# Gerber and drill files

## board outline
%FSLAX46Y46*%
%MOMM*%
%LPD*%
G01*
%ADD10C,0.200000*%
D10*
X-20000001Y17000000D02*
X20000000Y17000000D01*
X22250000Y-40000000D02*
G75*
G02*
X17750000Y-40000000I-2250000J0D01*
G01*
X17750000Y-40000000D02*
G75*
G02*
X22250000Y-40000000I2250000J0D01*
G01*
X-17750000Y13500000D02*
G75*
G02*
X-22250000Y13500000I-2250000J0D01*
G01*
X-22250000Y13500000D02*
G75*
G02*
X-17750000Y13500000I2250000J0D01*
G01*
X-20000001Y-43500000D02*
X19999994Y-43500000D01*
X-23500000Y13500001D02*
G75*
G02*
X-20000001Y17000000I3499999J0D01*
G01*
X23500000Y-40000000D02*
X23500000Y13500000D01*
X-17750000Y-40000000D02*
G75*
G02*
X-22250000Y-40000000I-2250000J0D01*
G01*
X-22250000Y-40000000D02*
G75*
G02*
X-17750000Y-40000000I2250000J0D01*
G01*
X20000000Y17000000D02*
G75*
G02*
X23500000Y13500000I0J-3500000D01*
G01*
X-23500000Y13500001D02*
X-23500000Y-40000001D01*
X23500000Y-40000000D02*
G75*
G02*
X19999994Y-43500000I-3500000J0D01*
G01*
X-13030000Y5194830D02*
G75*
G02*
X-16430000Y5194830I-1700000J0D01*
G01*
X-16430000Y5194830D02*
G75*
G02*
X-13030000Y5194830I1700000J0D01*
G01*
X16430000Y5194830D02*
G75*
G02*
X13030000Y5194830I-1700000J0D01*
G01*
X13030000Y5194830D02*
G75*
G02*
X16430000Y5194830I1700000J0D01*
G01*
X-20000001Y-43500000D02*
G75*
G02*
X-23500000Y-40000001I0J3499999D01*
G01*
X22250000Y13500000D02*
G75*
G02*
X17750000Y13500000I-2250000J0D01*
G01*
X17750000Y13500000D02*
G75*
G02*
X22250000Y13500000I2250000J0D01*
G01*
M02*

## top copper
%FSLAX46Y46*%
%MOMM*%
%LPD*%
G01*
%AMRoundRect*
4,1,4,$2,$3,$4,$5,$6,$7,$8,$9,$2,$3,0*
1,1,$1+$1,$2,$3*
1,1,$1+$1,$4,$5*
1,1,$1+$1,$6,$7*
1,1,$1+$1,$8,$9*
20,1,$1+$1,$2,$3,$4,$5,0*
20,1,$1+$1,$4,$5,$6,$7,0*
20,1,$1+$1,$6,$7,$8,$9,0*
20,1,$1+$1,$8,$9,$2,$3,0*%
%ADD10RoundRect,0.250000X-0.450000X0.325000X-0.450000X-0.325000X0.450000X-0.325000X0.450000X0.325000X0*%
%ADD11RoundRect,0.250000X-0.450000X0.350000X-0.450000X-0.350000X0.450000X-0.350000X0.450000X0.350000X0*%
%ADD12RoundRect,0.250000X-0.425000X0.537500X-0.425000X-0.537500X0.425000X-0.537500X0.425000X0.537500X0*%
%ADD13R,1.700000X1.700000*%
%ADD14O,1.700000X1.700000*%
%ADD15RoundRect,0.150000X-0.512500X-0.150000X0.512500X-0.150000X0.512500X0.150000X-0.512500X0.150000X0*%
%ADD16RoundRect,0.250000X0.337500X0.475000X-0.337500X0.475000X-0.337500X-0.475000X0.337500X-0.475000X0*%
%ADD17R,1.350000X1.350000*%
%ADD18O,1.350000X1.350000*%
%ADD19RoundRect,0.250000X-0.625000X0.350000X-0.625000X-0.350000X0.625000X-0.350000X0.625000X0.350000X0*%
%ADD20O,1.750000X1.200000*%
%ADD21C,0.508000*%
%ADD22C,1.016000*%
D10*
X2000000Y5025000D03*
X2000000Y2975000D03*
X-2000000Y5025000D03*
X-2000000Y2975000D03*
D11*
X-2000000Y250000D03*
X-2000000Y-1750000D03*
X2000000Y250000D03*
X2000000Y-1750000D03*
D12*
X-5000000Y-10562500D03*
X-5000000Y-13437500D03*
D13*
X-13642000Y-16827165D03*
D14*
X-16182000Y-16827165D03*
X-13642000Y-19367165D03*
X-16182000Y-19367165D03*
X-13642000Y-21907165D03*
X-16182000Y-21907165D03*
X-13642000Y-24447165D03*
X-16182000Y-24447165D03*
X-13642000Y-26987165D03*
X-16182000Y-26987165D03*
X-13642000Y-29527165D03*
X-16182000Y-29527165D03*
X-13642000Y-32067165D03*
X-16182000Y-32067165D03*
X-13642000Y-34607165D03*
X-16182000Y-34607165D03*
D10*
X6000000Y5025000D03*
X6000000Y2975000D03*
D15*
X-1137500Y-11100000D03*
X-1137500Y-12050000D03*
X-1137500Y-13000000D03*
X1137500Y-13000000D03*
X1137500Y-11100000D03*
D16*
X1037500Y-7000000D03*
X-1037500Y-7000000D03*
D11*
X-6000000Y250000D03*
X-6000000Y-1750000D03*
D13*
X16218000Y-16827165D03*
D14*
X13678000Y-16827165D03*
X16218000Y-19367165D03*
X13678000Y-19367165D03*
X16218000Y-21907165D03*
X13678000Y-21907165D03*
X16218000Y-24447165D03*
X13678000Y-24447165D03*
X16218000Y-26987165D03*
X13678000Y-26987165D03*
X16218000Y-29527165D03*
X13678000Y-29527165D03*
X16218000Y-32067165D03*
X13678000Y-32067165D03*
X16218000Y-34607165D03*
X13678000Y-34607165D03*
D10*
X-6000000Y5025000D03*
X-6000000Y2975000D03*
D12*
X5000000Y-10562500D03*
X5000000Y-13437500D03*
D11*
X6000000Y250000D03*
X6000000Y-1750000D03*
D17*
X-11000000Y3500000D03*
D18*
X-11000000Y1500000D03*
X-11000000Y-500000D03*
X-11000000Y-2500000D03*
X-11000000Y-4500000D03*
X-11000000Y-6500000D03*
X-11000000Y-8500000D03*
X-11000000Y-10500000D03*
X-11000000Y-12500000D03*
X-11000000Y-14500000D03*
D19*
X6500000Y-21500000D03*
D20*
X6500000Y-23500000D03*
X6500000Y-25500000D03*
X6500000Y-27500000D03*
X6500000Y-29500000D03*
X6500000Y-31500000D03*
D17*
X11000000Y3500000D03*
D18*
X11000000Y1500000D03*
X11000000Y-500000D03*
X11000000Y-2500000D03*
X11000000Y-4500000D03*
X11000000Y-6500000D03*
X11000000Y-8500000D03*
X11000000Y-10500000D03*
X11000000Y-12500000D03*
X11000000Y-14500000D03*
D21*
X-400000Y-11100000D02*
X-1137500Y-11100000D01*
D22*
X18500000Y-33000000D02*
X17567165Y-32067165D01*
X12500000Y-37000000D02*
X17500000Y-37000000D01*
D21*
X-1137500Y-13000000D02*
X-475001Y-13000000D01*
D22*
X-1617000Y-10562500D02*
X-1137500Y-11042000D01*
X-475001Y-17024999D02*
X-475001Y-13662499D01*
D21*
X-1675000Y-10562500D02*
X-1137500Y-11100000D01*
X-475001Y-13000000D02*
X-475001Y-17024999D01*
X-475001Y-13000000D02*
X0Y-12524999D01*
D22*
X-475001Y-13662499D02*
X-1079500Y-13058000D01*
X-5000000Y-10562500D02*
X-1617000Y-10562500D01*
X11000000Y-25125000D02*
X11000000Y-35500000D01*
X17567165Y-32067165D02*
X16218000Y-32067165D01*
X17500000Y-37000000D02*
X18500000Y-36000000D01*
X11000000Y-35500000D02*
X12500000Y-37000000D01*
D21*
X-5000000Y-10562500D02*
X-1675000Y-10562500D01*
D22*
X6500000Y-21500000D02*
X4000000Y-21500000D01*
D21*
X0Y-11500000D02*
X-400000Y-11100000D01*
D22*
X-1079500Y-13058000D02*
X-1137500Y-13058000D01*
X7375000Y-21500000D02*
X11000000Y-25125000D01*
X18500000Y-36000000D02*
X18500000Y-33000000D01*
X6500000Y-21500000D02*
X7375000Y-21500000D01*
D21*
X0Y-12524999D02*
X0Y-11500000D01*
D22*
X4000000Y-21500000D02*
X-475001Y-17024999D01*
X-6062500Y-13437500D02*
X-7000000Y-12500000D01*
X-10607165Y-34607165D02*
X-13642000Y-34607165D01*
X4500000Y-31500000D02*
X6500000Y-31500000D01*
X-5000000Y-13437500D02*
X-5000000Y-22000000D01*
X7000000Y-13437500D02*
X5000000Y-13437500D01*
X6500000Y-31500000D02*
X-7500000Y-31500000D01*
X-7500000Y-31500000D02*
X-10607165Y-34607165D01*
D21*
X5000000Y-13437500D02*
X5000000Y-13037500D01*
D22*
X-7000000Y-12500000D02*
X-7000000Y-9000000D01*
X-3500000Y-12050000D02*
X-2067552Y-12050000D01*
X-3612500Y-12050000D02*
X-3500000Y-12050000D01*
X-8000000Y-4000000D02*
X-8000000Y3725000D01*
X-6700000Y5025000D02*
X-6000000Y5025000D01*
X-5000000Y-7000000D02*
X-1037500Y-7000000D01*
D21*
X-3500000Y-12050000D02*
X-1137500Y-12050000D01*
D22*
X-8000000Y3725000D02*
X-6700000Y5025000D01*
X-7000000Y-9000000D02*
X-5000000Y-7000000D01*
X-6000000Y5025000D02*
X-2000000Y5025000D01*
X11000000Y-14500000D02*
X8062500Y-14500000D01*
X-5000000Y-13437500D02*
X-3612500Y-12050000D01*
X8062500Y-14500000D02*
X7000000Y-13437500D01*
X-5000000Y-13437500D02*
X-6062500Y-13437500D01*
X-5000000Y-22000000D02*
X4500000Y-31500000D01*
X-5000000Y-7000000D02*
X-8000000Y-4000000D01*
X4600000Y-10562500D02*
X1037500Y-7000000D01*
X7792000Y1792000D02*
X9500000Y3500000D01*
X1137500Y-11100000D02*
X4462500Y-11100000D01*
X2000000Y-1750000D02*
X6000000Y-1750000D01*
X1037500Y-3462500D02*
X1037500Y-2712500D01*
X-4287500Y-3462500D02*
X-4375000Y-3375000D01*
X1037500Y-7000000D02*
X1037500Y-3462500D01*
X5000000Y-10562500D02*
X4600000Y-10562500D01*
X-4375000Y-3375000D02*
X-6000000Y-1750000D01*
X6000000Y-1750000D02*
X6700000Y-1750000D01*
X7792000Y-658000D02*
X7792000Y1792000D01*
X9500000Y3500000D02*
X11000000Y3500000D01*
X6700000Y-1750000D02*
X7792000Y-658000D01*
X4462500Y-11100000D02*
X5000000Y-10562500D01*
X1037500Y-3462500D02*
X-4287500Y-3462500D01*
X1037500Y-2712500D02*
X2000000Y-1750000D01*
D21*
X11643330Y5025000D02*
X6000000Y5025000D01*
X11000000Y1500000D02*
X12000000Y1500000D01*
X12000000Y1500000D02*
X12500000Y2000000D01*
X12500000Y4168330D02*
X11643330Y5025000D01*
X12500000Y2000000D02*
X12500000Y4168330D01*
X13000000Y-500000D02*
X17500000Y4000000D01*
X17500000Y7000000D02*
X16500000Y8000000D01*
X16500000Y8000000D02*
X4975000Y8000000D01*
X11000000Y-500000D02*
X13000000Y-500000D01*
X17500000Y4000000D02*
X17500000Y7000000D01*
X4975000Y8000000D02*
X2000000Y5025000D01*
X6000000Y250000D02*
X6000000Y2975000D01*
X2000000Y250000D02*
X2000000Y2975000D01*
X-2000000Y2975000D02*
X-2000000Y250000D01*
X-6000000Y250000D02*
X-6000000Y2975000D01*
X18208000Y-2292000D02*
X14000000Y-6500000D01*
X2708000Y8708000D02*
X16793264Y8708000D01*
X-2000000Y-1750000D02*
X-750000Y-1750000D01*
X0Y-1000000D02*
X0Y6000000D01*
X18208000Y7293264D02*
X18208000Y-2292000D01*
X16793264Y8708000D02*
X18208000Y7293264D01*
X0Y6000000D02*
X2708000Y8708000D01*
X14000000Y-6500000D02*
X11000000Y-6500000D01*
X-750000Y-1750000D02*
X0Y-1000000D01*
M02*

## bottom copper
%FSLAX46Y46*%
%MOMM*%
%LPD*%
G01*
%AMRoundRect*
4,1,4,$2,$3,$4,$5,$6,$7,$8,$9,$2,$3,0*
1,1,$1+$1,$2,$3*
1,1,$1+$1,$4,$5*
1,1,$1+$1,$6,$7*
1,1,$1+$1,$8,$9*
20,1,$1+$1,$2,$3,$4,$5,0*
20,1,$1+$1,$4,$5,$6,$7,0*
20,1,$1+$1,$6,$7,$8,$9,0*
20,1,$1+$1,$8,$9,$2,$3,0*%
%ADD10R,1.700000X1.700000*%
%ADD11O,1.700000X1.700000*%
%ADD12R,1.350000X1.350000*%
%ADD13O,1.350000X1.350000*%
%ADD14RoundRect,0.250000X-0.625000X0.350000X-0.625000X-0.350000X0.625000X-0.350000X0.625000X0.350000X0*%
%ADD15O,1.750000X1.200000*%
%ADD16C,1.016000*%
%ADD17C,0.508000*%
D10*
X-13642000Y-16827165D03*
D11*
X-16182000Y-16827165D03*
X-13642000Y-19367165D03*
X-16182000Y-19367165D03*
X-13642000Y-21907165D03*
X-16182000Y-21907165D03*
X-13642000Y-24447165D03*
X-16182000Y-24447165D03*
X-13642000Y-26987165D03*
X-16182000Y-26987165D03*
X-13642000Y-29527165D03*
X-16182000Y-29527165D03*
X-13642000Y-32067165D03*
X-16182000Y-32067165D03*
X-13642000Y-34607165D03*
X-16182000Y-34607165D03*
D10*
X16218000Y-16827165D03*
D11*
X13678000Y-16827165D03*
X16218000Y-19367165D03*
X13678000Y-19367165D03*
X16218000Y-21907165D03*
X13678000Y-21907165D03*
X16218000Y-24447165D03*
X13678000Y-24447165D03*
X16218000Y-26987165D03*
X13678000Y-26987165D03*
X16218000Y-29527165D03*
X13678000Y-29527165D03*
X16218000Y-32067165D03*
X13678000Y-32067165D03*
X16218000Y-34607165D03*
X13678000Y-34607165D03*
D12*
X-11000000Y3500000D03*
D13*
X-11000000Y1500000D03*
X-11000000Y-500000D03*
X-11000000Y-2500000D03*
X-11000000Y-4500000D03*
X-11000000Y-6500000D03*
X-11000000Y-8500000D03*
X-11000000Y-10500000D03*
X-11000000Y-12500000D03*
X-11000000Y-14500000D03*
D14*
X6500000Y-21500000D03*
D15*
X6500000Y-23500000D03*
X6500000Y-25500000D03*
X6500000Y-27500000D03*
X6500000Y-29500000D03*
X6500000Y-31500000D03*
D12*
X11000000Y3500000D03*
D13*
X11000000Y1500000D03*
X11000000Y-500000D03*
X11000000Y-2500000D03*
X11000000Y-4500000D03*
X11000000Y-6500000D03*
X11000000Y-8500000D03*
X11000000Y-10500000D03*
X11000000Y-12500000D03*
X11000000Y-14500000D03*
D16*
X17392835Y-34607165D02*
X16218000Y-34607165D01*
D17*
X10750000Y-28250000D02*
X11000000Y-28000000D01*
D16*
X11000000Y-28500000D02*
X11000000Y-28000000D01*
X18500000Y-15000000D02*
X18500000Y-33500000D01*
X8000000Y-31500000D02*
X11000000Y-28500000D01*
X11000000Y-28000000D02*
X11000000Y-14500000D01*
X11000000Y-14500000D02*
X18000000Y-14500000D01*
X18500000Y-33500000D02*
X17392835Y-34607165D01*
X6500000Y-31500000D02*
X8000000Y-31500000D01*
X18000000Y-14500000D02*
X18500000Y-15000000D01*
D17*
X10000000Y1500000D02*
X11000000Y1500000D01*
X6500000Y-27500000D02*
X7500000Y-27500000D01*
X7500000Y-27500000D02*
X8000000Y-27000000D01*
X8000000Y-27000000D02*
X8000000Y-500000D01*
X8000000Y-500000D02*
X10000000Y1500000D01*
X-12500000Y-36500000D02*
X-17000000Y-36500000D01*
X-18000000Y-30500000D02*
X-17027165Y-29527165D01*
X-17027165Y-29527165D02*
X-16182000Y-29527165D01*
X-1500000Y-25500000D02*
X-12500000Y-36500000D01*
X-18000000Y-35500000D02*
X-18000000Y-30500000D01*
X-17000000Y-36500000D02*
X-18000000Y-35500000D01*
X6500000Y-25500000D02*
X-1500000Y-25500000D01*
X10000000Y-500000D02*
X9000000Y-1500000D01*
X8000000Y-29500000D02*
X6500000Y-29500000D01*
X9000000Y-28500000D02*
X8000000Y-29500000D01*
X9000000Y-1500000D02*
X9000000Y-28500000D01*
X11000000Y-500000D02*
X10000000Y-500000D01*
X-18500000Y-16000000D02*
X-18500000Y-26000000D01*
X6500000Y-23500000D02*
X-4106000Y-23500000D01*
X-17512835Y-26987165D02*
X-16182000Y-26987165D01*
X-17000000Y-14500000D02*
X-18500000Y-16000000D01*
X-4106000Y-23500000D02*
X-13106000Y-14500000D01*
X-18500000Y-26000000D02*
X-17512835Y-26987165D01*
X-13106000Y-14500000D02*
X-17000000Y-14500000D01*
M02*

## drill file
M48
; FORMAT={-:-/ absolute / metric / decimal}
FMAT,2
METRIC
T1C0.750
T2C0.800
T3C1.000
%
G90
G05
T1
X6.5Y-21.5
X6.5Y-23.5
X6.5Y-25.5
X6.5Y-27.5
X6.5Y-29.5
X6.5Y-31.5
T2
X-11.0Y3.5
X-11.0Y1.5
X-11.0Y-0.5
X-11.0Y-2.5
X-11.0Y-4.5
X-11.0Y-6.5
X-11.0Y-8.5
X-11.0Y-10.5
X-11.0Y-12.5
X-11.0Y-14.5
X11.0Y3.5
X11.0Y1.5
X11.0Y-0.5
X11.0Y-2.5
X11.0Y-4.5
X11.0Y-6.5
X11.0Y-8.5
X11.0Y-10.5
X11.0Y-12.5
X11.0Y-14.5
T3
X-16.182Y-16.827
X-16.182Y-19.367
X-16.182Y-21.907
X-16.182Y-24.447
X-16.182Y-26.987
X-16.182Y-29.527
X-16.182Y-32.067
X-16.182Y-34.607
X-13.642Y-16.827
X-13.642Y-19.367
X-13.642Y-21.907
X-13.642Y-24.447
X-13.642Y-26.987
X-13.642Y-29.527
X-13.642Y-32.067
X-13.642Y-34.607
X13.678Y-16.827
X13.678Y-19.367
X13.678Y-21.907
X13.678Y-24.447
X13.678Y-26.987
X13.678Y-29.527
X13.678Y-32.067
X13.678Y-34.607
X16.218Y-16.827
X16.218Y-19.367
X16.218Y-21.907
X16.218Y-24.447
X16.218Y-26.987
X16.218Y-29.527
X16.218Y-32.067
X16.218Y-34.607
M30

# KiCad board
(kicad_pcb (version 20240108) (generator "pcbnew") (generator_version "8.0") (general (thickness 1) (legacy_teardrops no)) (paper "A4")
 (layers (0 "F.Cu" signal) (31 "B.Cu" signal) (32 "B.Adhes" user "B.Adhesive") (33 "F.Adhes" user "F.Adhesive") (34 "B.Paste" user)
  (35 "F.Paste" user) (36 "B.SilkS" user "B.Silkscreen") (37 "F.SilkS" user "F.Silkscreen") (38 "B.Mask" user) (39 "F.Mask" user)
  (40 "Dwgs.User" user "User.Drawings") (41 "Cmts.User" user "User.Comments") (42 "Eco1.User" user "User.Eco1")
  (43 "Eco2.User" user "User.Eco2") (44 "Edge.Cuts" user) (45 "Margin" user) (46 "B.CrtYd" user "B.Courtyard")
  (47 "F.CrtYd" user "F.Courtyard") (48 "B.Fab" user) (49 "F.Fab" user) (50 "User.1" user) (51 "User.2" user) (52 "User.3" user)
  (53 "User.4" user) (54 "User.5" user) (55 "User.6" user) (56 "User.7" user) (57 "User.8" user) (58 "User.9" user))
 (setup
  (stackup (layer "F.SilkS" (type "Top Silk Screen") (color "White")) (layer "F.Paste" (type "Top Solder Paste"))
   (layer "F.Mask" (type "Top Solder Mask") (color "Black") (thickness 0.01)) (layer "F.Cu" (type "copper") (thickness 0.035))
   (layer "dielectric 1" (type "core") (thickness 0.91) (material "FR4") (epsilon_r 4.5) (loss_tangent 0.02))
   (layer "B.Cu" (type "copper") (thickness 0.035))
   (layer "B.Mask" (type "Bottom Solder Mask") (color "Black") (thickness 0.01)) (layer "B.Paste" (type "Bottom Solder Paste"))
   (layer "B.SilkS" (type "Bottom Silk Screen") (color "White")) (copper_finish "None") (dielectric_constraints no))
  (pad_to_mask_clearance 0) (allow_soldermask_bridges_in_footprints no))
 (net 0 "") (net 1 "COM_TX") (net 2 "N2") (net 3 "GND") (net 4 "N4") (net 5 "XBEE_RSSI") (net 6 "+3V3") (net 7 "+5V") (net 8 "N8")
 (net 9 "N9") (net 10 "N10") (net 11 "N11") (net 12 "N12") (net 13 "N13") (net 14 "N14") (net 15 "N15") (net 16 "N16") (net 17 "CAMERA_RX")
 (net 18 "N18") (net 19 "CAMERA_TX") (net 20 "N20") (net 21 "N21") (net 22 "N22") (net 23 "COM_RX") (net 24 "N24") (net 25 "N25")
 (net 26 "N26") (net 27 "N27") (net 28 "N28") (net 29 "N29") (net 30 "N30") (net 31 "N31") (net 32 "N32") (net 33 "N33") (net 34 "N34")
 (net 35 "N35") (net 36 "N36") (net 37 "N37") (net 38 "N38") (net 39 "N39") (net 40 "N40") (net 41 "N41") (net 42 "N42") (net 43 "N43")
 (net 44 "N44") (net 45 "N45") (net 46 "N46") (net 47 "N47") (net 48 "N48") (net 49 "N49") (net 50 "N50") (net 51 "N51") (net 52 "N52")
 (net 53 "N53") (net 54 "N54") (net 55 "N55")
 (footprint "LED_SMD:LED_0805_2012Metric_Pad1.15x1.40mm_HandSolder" (layer "F.Cu") (at 2 -4 -90)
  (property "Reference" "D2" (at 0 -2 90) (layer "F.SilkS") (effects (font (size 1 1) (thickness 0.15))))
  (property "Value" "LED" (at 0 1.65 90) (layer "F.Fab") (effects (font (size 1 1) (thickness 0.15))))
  (pad "1" smd roundrect (at -1.025 0 270) (size 1.15 1.4) (layers "F.Cu" "F.Paste" "F.Mask") (roundrect_rratio 0.217391) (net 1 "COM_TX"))
  (pad "2" smd roundrect (at 1.025 0 270) (size 1.15 1.4) (layers "F.Cu" "F.Paste" "F.Mask") (roundrect_rratio 0.217391) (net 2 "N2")))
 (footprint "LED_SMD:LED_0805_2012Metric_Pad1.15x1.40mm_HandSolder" (layer "F.Cu") (at -2 -4 -90)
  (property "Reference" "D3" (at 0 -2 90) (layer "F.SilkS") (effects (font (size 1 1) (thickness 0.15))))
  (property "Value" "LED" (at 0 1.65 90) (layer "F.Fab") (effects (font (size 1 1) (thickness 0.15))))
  (pad "1" smd roundrect (at -1.025 0 270) (size 1.15 1.4) (layers "F.Cu" "F.Paste" "F.Mask") (roundrect_rratio 0.217391) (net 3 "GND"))
  (pad "2" smd roundrect (at 1.025 0 270) (size 1.15 1.4) (layers "F.Cu" "F.Paste" "F.Mask") (roundrect_rratio 0.217391) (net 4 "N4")))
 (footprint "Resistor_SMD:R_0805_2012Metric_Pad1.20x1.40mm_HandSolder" (layer "F.Cu") (at -2 0.75 -90)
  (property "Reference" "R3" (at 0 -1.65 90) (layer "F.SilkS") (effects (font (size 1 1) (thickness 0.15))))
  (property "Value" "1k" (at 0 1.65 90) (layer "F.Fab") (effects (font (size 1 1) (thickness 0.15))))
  (pad "1" smd roundrect (at -1 0 270) (size 1.2 1.4) (layers "F.Cu" "F.Paste" "F.Mask") (roundrect_rratio 0.208333) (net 4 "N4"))
  (pad "2" smd roundrect (at 1 0 270) (size 1.2 1.4) (layers "F.Cu" "F.Paste" "F.Mask") (roundrect_rratio 0.208333) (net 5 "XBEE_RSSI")))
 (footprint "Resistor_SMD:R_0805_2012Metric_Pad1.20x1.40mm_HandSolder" (layer "F.Cu") (at 2 0.75 -90)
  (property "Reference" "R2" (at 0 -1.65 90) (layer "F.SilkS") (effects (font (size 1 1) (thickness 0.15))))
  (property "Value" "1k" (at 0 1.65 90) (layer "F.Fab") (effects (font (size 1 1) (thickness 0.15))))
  (pad "1" smd roundrect (at -1 0 270) (size 1.2 1.4) (layers "F.Cu" "F.Paste" "F.Mask") (roundrect_rratio 0.208333) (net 2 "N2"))
  (pad "2" smd roundrect (at 1 0 270) (size 1.2 1.4) (layers "F.Cu" "F.Paste" "F.Mask") (roundrect_rratio 0.208333) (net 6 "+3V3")))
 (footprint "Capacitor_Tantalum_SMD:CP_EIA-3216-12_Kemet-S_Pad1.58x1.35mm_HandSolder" (layer "F.Cu") (at -5 12 -90)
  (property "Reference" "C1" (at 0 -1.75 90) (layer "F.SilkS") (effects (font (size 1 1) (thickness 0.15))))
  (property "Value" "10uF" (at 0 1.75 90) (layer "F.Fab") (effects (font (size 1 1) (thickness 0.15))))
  (pad "1" smd roundrect (at -1.4375 0 270) (size 1.575 1.35) (layers "F.Cu" "F.Paste" "F.Mask") (roundrect_rratio 0.185185) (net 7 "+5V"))
  (pad "2" smd roundrect (at 1.4375 0 270) (size 1.575 1.35) (layers "F.Cu" "F.Paste" "F.Mask") (roundrect_rratio 0.185185) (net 3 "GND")))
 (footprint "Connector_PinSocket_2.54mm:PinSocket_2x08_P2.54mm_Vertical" (layer "F.Cu") (at -13.642 16.827165)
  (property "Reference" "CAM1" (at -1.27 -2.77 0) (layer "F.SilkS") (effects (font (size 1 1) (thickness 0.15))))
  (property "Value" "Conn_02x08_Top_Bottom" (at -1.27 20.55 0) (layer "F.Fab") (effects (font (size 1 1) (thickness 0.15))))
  (pad "1" thru_hole rect (at 0 0) (size 1.7 1.7) (drill 1) (layers "*.Cu" "*.Mask") (remove_unused_layers no) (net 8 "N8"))
  (pad "2" thru_hole oval (at -2.54 0) (size 1.7 1.7) (drill 1) (layers "*.Cu" "*.Mask") (remove_unused_layers no) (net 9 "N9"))
  (pad "3" thru_hole oval (at 0 2.54) (size 1.7 1.7) (drill 1) (layers "*.Cu" "*.Mask") (remove_unused_layers no) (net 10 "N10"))
  (pad "4" thru_hole oval (at -2.54 2.54) (size 1.7 1.7) (drill 1) (layers "*.Cu" "*.Mask") (remove_unused_layers no) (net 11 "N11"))
  (pad "5" thru_hole oval (at 0 5.08) (size 1.7 1.7) (drill 1) (layers "*.Cu" "*.Mask") (remove_unused_layers no) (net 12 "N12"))
  (pad "6" thru_hole oval (at -2.54 5.08) (size 1.7 1.7) (drill 1) (layers "*.Cu" "*.Mask") (remove_unused_layers no) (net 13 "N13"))
  (pad "7" thru_hole oval (at 0 7.62) (size 1.7 1.7) (drill 1) (layers "*.Cu" "*.Mask") (remove_unused_layers no) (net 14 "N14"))
  (pad "8" thru_hole oval (at -2.54 7.62) (size 1.7 1.7) (drill 1) (layers "*.Cu" "*.Mask") (remove_unused_layers no) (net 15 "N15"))
  (pad "9" thru_hole oval (at 0 10.16) (size 1.7 1.7) (drill 1) (layers "*.Cu" "*.Mask") (remove_unused_layers no) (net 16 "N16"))
  (pad "10" thru_hole oval (at -2.54 10.16) (size 1.7 1.7) (drill 1) (layers "*.Cu" "*.Mask") (remove_unused_layers no) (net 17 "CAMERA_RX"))
  (pad "11" thru_hole oval (at 0 12.7) (size 1.7 1.7) (drill 1) (layers "*.Cu" "*.Mask") (remove_unused_layers no) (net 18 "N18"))
  (pad "12" thru_hole oval (at -2.54 12.7) (size 1.7 1.7) (drill 1) (layers "*.Cu" "*.Mask") (remove_unused_layers no) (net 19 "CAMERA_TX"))
  (pad "13" thru_hole oval (at 0 15.24) (size 1.7 1.7) (drill 1) (layers "*.Cu" "*.Mask") (remove_unused_layers no) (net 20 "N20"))
  (pad "14" thru_hole oval (at -2.54 15.24) (size 1.7 1.7) (drill 1) (layers "*.Cu" "*.Mask") (remove_unused_layers no) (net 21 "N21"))
  (pad "15" thru_hole oval (at 0 17.78) (size 1.7 1.7) (drill 1) (layers "*.Cu" "*.Mask") (remove_unused_layers no) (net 3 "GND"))
  (pad "16" thru_hole oval (at -2.54 17.78) (size 1.7 1.7) (drill 1) (layers "*.Cu" "*.Mask") (remove_unused_layers no) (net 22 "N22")))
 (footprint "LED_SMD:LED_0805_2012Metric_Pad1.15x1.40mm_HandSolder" (layer "F.Cu") (at 6 -4 -90)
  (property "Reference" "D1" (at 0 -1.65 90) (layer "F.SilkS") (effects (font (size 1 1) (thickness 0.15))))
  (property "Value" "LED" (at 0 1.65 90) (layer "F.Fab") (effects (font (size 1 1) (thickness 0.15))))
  (pad "1" smd roundrect (at -1.025 0 270) (size 1.15 1.4) (layers "F.Cu" "F.Paste" "F.Mask") (roundrect_rratio 0.217391) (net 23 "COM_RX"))
  (pad "2" smd roundrect (at 1.025 0 270) (size 1.15 1.4) (layers "F.Cu" "F.Paste" "F.Mask") (roundrect_rratio 0.217391) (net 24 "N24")))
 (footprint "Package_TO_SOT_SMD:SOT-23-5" (layer "F.Cu") (at 0 12.05)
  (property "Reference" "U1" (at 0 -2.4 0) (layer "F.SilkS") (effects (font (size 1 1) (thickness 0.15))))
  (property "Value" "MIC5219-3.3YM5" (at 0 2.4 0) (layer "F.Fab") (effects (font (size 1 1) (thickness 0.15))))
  (pad "1" smd roundrect (at -1.1375 -0.95) (size 1.325 0.6) (layers "F.Cu" "F.Paste" "F.Mask") (roundrect_rratio 0.25) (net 7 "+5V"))
  (pad "2" smd roundrect (at -1.1375 0) (size 1.325 0.6) (layers "F.Cu" "F.Paste" "F.Mask") (roundrect_rratio 0.25) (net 3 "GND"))
  (pad "3" smd roundrect (at -1.1375 0.95) (size 1.325 0.6) (layers "F.Cu" "F.Paste" "F.Mask") (roundrect_rratio 0.25) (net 7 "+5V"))
  (pad "4" smd roundrect (at 1.1375 0.95) (size 1.325 0.6) (layers "F.Cu" "F.Paste" "F.Mask") (roundrect_rratio 0.25) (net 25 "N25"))
  (pad "5" smd roundrect (at 1.1375 -0.95) (size 1.325 0.6) (layers "F.Cu" "F.Paste" "F.Mask") (roundrect_rratio 0.25) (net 6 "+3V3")))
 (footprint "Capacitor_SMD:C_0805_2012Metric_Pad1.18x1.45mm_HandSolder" (layer "F.Cu") (at 0 7 180)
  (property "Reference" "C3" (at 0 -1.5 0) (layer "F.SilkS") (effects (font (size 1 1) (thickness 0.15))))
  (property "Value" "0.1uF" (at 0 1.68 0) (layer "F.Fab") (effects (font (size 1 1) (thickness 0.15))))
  (pad "1" smd roundrect (at -1.0375 0 180) (size 1.175 1.45) (layers "F.Cu" "F.Paste" "F.Mask") (roundrect_rratio 0.212766) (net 6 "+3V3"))
  (pad "2" smd roundrect (at 1.0375 0 180) (size 1.175 1.45) (layers "F.Cu" "F.Paste" "F.Mask") (roundrect_rratio 0.212766) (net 3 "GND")))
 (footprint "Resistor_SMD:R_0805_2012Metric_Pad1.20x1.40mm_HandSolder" (layer "F.Cu") (at -6 0.75 -90)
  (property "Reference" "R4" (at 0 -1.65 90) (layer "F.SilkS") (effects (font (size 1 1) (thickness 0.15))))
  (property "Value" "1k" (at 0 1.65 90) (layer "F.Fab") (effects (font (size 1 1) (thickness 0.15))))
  (pad "1" smd roundrect (at -1 0 270) (size 1.2 1.4) (layers "F.Cu" "F.Paste" "F.Mask") (roundrect_rratio 0.208333) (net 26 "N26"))
  (pad "2" smd roundrect (at 1 0 270) (size 1.2 1.4) (layers "F.Cu" "F.Paste" "F.Mask") (roundrect_rratio 0.208333) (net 6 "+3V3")))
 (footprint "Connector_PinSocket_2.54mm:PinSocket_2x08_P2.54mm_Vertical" (layer "F.Cu") (at 16.218 16.827165)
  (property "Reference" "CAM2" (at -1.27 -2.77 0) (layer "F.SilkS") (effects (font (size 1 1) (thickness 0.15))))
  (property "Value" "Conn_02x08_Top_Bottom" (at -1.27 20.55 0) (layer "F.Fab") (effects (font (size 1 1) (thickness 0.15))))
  (pad "1" thru_hole rect (at 0 0) (size 1.7 1.7) (drill 1) (layers "*.Cu" "*.Mask") (remove_unused_layers no) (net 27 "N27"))
  (pad "2" thru_hole oval (at -2.54 0) (size 1.7 1.7) (drill 1) (layers "*.Cu" "*.Mask") (remove_unused_layers no) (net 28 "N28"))
  (pad "3" thru_hole oval (at 0 2.54) (size 1.7 1.7) (drill 1) (layers "*.Cu" "*.Mask") (remove_unused_layers no) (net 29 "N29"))
  (pad "4" thru_hole oval (at -2.54 2.54) (size 1.7 1.7) (drill 1) (layers "*.Cu" "*.Mask") (remove_unused_layers no) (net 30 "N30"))
  (pad "5" thru_hole oval (at 0 5.08) (size 1.7 1.7) (drill 1) (layers "*.Cu" "*.Mask") (remove_unused_layers no) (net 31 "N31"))
  (pad "6" thru_hole oval (at -2.54 5.08) (size 1.7 1.7) (drill 1) (layers "*.Cu" "*.Mask") (remove_unused_layers no) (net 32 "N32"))
  (pad "7" thru_hole oval (at 0 7.62) (size 1.7 1.7) (drill 1) (layers "*.Cu" "*.Mask") (remove_unused_layers no) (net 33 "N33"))
  (pad "8" thru_hole oval (at -2.54 7.62) (size 1.7 1.7) (drill 1) (layers "*.Cu" "*.Mask") (remove_unused_layers no) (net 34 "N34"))
  (pad "9" thru_hole oval (at 0 10.16) (size 1.7 1.7) (drill 1) (layers "*.Cu" "*.Mask") (remove_unused_layers no) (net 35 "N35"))
  (pad "10" thru_hole oval (at -2.54 10.16) (size 1.7 1.7) (drill 1) (layers "*.Cu" "*.Mask") (remove_unused_layers no) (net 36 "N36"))
  (pad "11" thru_hole oval (at 0 12.7) (size 1.7 1.7) (drill 1) (layers "*.Cu" "*.Mask") (remove_unused_layers no) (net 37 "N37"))
  (pad "12" thru_hole oval (at -2.54 12.7) (size 1.7 1.7) (drill 1) (layers "*.Cu" "*.Mask") (remove_unused_layers no) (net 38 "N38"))
  (pad "13" thru_hole oval (at 0 15.24) (size 1.7 1.7) (drill 1) (layers "*.Cu" "*.Mask") (remove_unused_layers no) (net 7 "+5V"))
  (pad "14" thru_hole oval (at -2.54 15.24) (size 1.7 1.7) (drill 1) (layers "*.Cu" "*.Mask") (remove_unused_layers no) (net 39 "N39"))
  (pad "15" thru_hole oval (at 0 17.78) (size 1.7 1.7) (drill 1) (layers "*.Cu" "*.Mask") (remove_unused_layers no) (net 3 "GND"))
  (pad "16" thru_hole oval (at -2.54 17.78) (size 1.7 1.7) (drill 1) (layers "*.Cu" "*.Mask") (remove_unused_layers no) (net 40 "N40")))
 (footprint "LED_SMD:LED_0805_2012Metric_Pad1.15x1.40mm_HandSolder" (layer "F.Cu") (at -6 -4 -90)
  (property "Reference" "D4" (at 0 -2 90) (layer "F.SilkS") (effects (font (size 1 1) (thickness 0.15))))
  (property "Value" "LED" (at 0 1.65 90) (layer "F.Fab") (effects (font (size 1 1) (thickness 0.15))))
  (pad "1" smd roundrect (at -1.025 0 270) (size 1.15 1.4) (layers "F.Cu" "F.Paste" "F.Mask") (roundrect_rratio 0.217391) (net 3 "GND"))
  (pad "2" smd roundrect (at 1.025 0 270) (size 1.15 1.4) (layers "F.Cu" "F.Paste" "F.Mask") (roundrect_rratio 0.217391) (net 26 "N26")))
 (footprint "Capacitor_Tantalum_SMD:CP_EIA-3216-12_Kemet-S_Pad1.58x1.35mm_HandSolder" (layer "F.Cu") (at 5 12 -90)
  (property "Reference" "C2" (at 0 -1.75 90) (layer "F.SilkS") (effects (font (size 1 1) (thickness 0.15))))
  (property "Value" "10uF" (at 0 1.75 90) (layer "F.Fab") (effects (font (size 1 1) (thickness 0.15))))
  (pad "1" smd roundrect (at -1.4375 0 270) (size 1.575 1.35) (layers "F.Cu" "F.Paste" "F.Mask") (roundrect_rratio 0.185185) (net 6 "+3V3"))
  (pad "2" smd roundrect (at 1.4375 0 270) (size 1.575 1.35) (layers "F.Cu" "F.Paste" "F.Mask") (roundrect_rratio 0.185185) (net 3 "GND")))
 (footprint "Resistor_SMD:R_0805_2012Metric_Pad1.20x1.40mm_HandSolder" (layer "F.Cu") (at 6 0.75 -90)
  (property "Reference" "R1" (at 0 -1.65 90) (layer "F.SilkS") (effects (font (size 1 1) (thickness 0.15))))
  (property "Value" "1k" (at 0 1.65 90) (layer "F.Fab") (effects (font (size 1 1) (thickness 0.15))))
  (pad "1" smd roundrect (at -1 0 270) (size 1.2 1.4) (layers "F.Cu" "F.Paste" "F.Mask") (roundrect_rratio 0.208333) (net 24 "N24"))
  (pad "2" smd roundrect (at 1 0 270) (size 1.2 1.4) (layers "F.Cu" "F.Paste" "F.Mask") (roundrect_rratio 0.208333) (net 6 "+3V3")))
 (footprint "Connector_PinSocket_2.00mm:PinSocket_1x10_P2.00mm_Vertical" (layer "B.Cu") (at -11 -3.5 180)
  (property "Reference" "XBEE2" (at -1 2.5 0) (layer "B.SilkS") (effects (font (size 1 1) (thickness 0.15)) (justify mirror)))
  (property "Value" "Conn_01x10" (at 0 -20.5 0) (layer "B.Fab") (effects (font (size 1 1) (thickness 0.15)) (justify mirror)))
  (pad "1" thru_hole rect (at 0 0 180) (size 1.35 1.35) (drill 0.8) (layers "*.Cu" "*.Mask") (remove_unused_layers no) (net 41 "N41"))
  (pad "2" thru_hole oval (at 0 -2 180) (size 1.35 1.35) (drill 0.8) (layers "*.Cu" "*.Mask") (remove_unused_layers no) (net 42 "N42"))
  (pad "3" thru_hole oval (at 0 -4 180) (size 1.35 1.35) (drill 0.8) (layers "*.Cu" "*.Mask") (remove_unused_layers no) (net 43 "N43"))
  (pad "4" thru_hole oval (at 0 -6 180) (size 1.35 1.35) (drill 0.8) (layers "*.Cu" "*.Mask") (remove_unused_layers no) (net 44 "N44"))
  (pad "5" thru_hole oval (at 0 -8 180) (size 1.35 1.35) (drill 0.8) (layers "*.Cu" "*.Mask") (remove_unused_layers no) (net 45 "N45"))
  (pad "6" thru_hole oval (at 0 -10 180) (size 1.35 1.35) (drill 0.8) (layers "*.Cu" "*.Mask") (remove_unused_layers no) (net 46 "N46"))
  (pad "7" thru_hole oval (at 0 -12 180) (size 1.35 1.35) (drill 0.8) (layers "*.Cu" "*.Mask") (remove_unused_layers no) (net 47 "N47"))
  (pad "8" thru_hole oval (at 0 -14 180) (size 1.35 1.35) (drill 0.8) (layers "*.Cu" "*.Mask") (remove_unused_layers no) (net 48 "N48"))
  (pad "9" thru_hole oval (at 0 -16 180) (size 1.35 1.35) (drill 0.8) (layers "*.Cu" "*.Mask") (remove_unused_layers no) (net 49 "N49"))
  (pad "10" thru_hole oval (at 0 -18 180) (size 1.35 1.35) (drill 0.8) (layers "*.Cu" "*.Mask") (remove_unused_layers no) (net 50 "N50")))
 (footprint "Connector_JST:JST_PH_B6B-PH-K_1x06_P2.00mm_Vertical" (layer "B.Cu") (at 6.5 21.5 -90)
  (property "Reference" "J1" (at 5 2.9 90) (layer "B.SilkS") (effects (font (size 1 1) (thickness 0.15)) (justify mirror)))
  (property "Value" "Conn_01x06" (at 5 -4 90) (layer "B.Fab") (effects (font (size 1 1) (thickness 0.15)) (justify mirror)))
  (pad "1" thru_hole roundrect (at 0 0 270) (size 1.2 1.75) (drill 0.75) (layers "*.Cu" "*.Mask") (remove_unused_layers no)
   (roundrect_rratio 0.208333) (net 7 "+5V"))
  (pad "2" thru_hole oval (at 2 0 270) (size 1.2 1.75) (drill 0.75) (layers "*.Cu" "*.Mask") (remove_unused_layers no) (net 17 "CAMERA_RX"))
  (pad "3" thru_hole oval (at 4 0 270) (size 1.2 1.75) (drill 0.75) (layers "*.Cu" "*.Mask") (remove_unused_layers no) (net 19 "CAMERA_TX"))
  (pad "4" thru_hole oval (at 6 0 270) (size 1.2 1.75) (drill 0.75) (layers "*.Cu" "*.Mask") (remove_unused_layers no) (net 23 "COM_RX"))
  (pad "5" thru_hole oval (at 8 0 270) (size 1.2 1.75) (drill 0.75) (layers "*.Cu" "*.Mask") (remove_unused_layers no) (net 1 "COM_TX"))
  (pad "6" thru_hole oval (at 10 0 270) (size 1.2 1.75) (drill 0.75) (layers "*.Cu" "*.Mask") (remove_unused_layers no) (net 3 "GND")))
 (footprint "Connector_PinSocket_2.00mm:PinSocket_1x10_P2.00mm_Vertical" (layer "B.Cu") (at 11 -3.5 180)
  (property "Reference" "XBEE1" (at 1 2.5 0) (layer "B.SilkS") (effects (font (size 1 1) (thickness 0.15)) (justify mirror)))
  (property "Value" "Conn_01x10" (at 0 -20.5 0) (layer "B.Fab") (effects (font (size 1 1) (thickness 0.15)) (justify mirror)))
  (pad "1" thru_hole rect (at 0 0 180) (size 1.35 1.35) (drill 0.8) (layers "*.Cu" "*.Mask") (remove_unused_layers no) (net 6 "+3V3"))
  (pad "2" thru_hole oval (at 0 -2 180) (size 1.35 1.35) (drill 0.8) (layers "*.Cu" "*.Mask") (remove_unused_layers no) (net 23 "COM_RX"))
  (pad "3" thru_hole oval (at 0 -4 180) (size 1.35 1.35) (drill 0.8) (layers "*.Cu" "*.Mask") (remove_unused_layers no) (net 1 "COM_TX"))
  (pad "4" thru_hole oval (at 0 -6 180) (size 1.35 1.35) (drill 0.8) (layers "*.Cu" "*.Mask") (remove_unused_layers no) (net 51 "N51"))
  (pad "5" thru_hole oval (at 0 -8 180) (size 1.35 1.35) (drill 0.8) (layers "*.Cu" "*.Mask") (remove_unused_layers no) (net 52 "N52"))
  (pad "6" thru_hole oval (at 0 -10 180) (size 1.35 1.35) (drill 0.8) (layers "*.Cu" "*.Mask") (remove_unused_layers no) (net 5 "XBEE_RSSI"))
  (pad "7" thru_hole oval (at 0 -12 180) (size 1.35 1.35) (drill 0.8) (layers "*.Cu" "*.Mask") (remove_unused_layers no) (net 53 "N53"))
  (pad "8" thru_hole oval (at 0 -14 180) (size 1.35 1.35) (drill 0.8) (layers "*.Cu" "*.Mask") (remove_unused_layers no) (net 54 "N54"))
  (pad "9" thru_hole oval (at 0 -16 180) (size 1.35 1.35) (drill 0.8) (layers "*.Cu" "*.Mask") (remove_unused_layers no) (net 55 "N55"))
  (pad "10" thru_hole oval (at 0 -18 180) (size 1.35 1.35) (drill 0.8) (layers "*.Cu" "*.Mask") (remove_unused_layers no) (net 3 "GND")))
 (gr_line (start -20.000001 -17) (end 20 -17) (stroke (width 0.2) (type default)) (layer "Edge.Cuts"))
 (gr_circle (center 20 40) (end 22.25 40) (stroke (width 0.2) (type default)) (fill none) (layer "Edge.Cuts"))
 (gr_circle (center -20 -13.5) (end -17.75 -13.5) (stroke (width 0.2) (type default)) (fill none) (layer "Edge.Cuts"))
 (gr_line (start -20.000001 43.5) (end 19.999994 43.5) (stroke (width 0.2) (type default)) (layer "Edge.Cuts"))
 (gr_arc (start -23.5 -13.500001) (mid -22.474874 -15.974874) (end -20.000001 -17) (stroke (width 0.2) (type default)) (layer "Edge.Cuts"))
 (gr_line (start 23.5 40) (end 23.5 -13.5) (stroke (width 0.2) (type default)) (layer "Edge.Cuts"))
 (gr_circle (center -20 40) (end -17.75 40) (stroke (width 0.2) (type default)) (fill none) (layer "Edge.Cuts"))
 (gr_arc (start 20 -17) (mid 22.474874 -15.974874) (end 23.5 -13.5) (stroke (width 0.2) (type default)) (layer "Edge.Cuts"))
 (gr_line (start -23.5 -13.500001) (end -23.5 40.000001) (stroke (width 0.2) (type default)) (layer "Edge.Cuts"))
 (gr_arc (start 23.5 40) (mid 22.474872 42.474876) (end 19.999994 43.5) (stroke (width 0.2) (type default)) (layer "Edge.Cuts"))
 (gr_circle (center -14.73 -5.19483) (end -13.03 -5.19483) (stroke (width 0.2) (type default)) (fill none) (layer "Edge.Cuts"))
 (gr_circle (center 14.73 -5.19483) (end 16.43 -5.19483) (stroke (width 0.2) (type default)) (fill none) (layer "Edge.Cuts"))
 (gr_arc (start -20.000001 43.5) (mid -22.474874 42.474874) (end -23.5 40.000001) (stroke (width 0.2) (type default)) (layer "Edge.Cuts"))
 (gr_circle (center 20 -13.5) (end 22.25 -13.5) (stroke (width 0.2) (type default)) (fill none) (layer "Edge.Cuts"))
 (segment (start -0.4 11.1) (end -1.1375 11.1) (width 0.508) (layer "F.Cu") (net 7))
 (segment (start 18.5 33) (end 17.567165 32.067165) (width 1.016) (layer "F.Cu") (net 7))
 (segment (start 12.5 37) (end 17.5 37) (width 1.016) (layer "F.Cu") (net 7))
 (segment (start -1.1375 13) (end -0.475001 13) (width 0.508) (layer "F.Cu") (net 7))
 (segment (start -1.617 10.5625) (end -1.1375 11.042) (width 1.016) (layer "F.Cu") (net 7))
 (segment (start -0.475001 17.024999) (end -0.475001 13.662499) (width 1.016) (layer "F.Cu") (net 7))
 (segment (start -1.675 10.5625) (end -1.1375 11.1) (width 0.508) (layer "F.Cu") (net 7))
 (segment (start -0.475001 13) (end -0.475001 17.024999) (width 0.508) (layer "F.Cu") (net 7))
 (segment (start -0.475001 13) (end 0 12.524999) (width 0.508) (layer "F.Cu") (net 7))
 (segment (start -0.475001 13.662499) (end -1.0795 13.058) (width 1.016) (layer "F.Cu") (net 7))
 (segment (start -5 10.5625) (end -1.617 10.5625) (width 1.016) (layer "F.Cu") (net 7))
 (segment (start 11 25.125) (end 11 35.5) (width 1.016) (layer "F.Cu") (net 7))
 (segment (start 17.567165 32.067165) (end 16.218 32.067165) (width 1.016) (layer "F.Cu") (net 7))
 (segment (start 17.5 37) (end 18.5 36) (width 1.016) (layer "F.Cu") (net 7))
 (segment (start 11 35.5) (end 12.5 37) (width 1.016) (layer "F.Cu") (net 7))
 (segment (start -5 10.5625) (end -1.675 10.5625) (width 0.508) (layer "F.Cu") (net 7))
 (segment (start 6.5 21.5) (end 4 21.5) (width 1.016) (layer "F.Cu") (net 7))
 (segment (start 0 11.5) (end -0.4 11.1) (width 0.508) (layer "F.Cu") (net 7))
 (segment (start -1.0795 13.058) (end -1.1375 13.058) (width 1.016) (layer "F.Cu") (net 7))
 (segment (start 7.375 21.5) (end 11 25.125) (width 1.016) (layer "F.Cu") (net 7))
 (segment (start 18.5 36) (end 18.5 33) (width 1.016) (layer "F.Cu") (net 7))
 (segment (start 6.5 21.5) (end 7.375 21.5) (width 1.016) (layer "F.Cu") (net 7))
 (segment (start 0 12.524999) (end 0 11.5) (width 0.508) (layer "F.Cu") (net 7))
 (segment (start 4 21.5) (end -0.475001 17.024999) (width 1.016) (layer "F.Cu") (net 7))
 (segment (start -6.0625 13.4375) (end -7 12.5) (width 1.016) (layer "F.Cu") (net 3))
 (segment (start -10.607165 34.607165) (end -13.642 34.607165) (width 1.016) (layer "F.Cu") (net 3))
 (segment (start 4.5 31.5) (end 6.5 31.5) (width 1.016) (layer "F.Cu") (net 3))
 (segment (start -5 13.4375) (end -5 22) (width 1.016) (layer "F.Cu") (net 3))
 (segment (start 7 13.4375) (end 5 13.4375) (width 1.016) (layer "F.Cu") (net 3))
 (segment (start 6.5 31.5) (end -7.5 31.5) (width 1.016) (layer "F.Cu") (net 3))
 (segment (start -7.5 31.5) (end -10.607165 34.607165) (width 1.016) (layer "F.Cu") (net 3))
 (segment (start 5 13.4375) (end 5 13.0375) (width 0.508) (layer "F.Cu") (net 3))
 (segment (start -7 12.5) (end -7 9) (width 1.016) (layer "F.Cu") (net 3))
 (segment (start -3.5 12.05) (end -2.067552 12.05) (width 1.016) (layer "F.Cu") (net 3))
 (segment (start -3.6125 12.05) (end -3.5 12.05) (width 1.016) (layer "F.Cu") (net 3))
 (segment (start -8 4) (end -8 -3.725) (width 1.016) (layer "F.Cu") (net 3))
 (segment (start -6.7 -5.025) (end -6 -5.025) (width 1.016) (layer "F.Cu") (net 3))
 (segment (start -5 7) (end -1.0375 7) (width 1.016) (layer "F.Cu") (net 3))
 (segment (start -3.5 12.05) (end -1.1375 12.05) (width 0.508) (layer "F.Cu") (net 3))
 (segment (start -8 -3.725) (end -6.7 -5.025) (width 1.016) (layer "F.Cu") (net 3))
 (segment (start -7 9) (end -5 7) (width 1.016) (layer "F.Cu") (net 3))
 (segment (start -6 -5.025) (end -2 -5.025) (width 1.016) (layer "F.Cu") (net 3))
 (segment (start 11 14.5) (end 8.0625 14.5) (width 1.016) (layer "F.Cu") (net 3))
 (segment (start -5 13.4375) (end -3.6125 12.05) (width 1.016) (layer "F.Cu") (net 3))
 (segment (start 8.0625 14.5) (end 7 13.4375) (width 1.016) (layer "F.Cu") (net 3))
 (segment (start -5 13.4375) (end -6.0625 13.4375) (width 1.016) (layer "F.Cu") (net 3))
 (segment (start -5 22) (end 4.5 31.5) (width 1.016) (layer "F.Cu") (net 3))
 (segment (start -5 7) (end -8 4) (width 1.016) (layer "F.Cu") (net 3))
 (segment (start 17.392835 34.607165) (end 16.218 34.607165) (width 1.016) (layer "B.Cu") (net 3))
 (segment (start 10.75 28.25) (end 11 28) (width 0.508) (layer "B.Cu") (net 3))
 (segment (start 11 28.5) (end 11 28) (width 1.016) (layer "B.Cu") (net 3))
 (segment (start 18.5 15) (end 18.5 33.5) (width 1.016) (layer "B.Cu") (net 3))
 (segment (start 8 31.5) (end 11 28.5) (width 1.016) (layer "B.Cu") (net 3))
 (segment (start 11 28) (end 11 14.5) (width 1.016) (layer "B.Cu") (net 3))
 (segment (start 11 14.5) (end 18 14.5) (width 1.016) (layer "B.Cu") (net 3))
 (segment (start 18.5 33.5) (end 17.392835 34.607165) (width 1.016) (layer "B.Cu") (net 3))
 (segment (start 6.5 31.5) (end 8 31.5) (width 1.016) (layer "B.Cu") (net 3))
 (segment (start 18 14.5) (end 18.5 15) (width 1.016) (layer "B.Cu") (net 3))
 (segment (start 4.6 10.5625) (end 1.0375 7) (width 1.016) (layer "F.Cu") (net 6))
 (segment (start 7.792 -1.792) (end 9.5 -3.5) (width 1.016) (layer "F.Cu") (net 6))
 (segment (start 1.1375 11.1) (end 4.4625 11.1) (width 1.016) (layer "F.Cu") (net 6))
 (segment (start 2 1.75) (end 6 1.75) (width 1.016) (layer "F.Cu") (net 6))
 (segment (start 1.0375 3.4625) (end 1.0375 2.7125) (width 1.016) (layer "F.Cu") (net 6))
 (segment (start -4.2875 3.4625) (end -4.375 3.375) (width 1.016) (layer "F.Cu") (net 6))
 (segment (start 1.0375 7) (end 1.0375 3.4625) (width 1.016) (layer "F.Cu") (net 6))
 (segment (start 5 10.5625) (end 4.6 10.5625) (width 1.016) (layer "F.Cu") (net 6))
 (segment (start -4.375 3.375) (end -6 1.75) (width 1.016) (layer "F.Cu") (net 6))
 (segment (start 6 1.75) (end 6.7 1.75) (width 1.016) (layer "F.Cu") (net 6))
 (segment (start 7.792 0.658) (end 7.792 -1.792) (width 1.016) (layer "F.Cu") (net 6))
 (segment (start 9.5 -3.5) (end 11 -3.5) (width 1.016) (layer "F.Cu") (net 6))
 (segment (start 6.7 1.75) (end 7.792 0.658) (width 1.016) (layer "F.Cu") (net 6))
 (segment (start 4.4625 11.1) (end 5 10.5625) (width 1.016) (layer "F.Cu") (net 6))
 (segment (start 1.0375 3.4625) (end -4.2875 3.4625) (width 1.016) (layer "F.Cu") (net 6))
 (segment (start 1.0375 2.7125) (end 2 1.75) (width 1.016) (layer "F.Cu") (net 6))
 (segment (start 11.64333 -5.025) (end 6 -5.025) (width 0.508) (layer "F.Cu") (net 23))
 (segment (start 11 -1.5) (end 12 -1.5) (width 0.508) (layer "F.Cu") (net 23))
 (segment (start 12 -1.5) (end 12.5 -2) (width 0.508) (layer "F.Cu") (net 23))
 (segment (start 12.5 -4.16833) (end 11.64333 -5.025) (width 0.508) (layer "F.Cu") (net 23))
 (segment (start 12.5 -2) (end 12.5 -4.16833) (width 0.508) (layer "F.Cu") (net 23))
 (segment (start 10 -1.5) (end 11 -1.5) (width 0.508) (layer "B.Cu") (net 23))
 (segment (start 6.5 27.5) (end 7.5 27.5) (width 0.508) (layer "B.Cu") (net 23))
 (segment (start 7.5 27.5) (end 8 27) (width 0.508) (layer "B.Cu") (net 23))
 (segment (start 8 27) (end 8 0.5) (width 0.508) (layer "B.Cu") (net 23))
 (segment (start 8 0.5) (end 10 -1.5) (width 0.508) (layer "B.Cu") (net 23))
 (segment (start -12.5 36.5) (end -17 36.5) (width 0.508) (layer "B.Cu") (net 19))
 (segment (start -18 30.5) (end -17.027165 29.527165) (width 0.508) (layer "B.Cu") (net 19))
 (segment (start -17.027165 29.527165) (end -16.182 29.527165) (width 0.508) (layer "B.Cu") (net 19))
 (segment (start -1.5 25.5) (end -12.5 36.5) (width 0.508) (layer "B.Cu") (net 19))
 (segment (start -18 35.5) (end -18 30.5) (width 0.508) (layer "B.Cu") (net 19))
 (segment (start -17 36.5) (end -18 35.5) (width 0.508) (layer "B.Cu") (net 19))
 (segment (start 6.5 25.5) (end -1.5 25.5) (width 0.508) (layer "B.Cu") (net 19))
 (segment (start 13 0.5) (end 17.5 -4) (width 0.508) (layer "F.Cu") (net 1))
 (segment (start 17.5 -7) (end 16.5 -8) (width 0.508) (layer "F.Cu") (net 1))
 (segment (start 16.5 -8) (end 4.975 -8) (width 0.508) (layer "F.Cu") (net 1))
 (segment (start 11 0.5) (end 13 0.5) (width 0.508) (layer "F.Cu") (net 1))
 (segment (start 17.5 -4) (end 17.5 -7) (width 0.508) (layer "F.Cu") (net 1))
 (segment (start 4.975 -8) (end 2 -5.025) (width 0.508) (layer "F.Cu") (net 1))
 (segment (start 10 0.5) (end 9 1.5) (width 0.508) (layer "B.Cu") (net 1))
 (segment (start 8 29.5) (end 6.5 29.5) (width 0.508) (layer "B.Cu") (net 1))
 (segment (start 9 28.5) (end 8 29.5) (width 0.508) (layer "B.Cu") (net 1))
 (segment (start 9 1.5) (end 9 28.5) (width 0.508) (layer "B.Cu") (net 1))
 (segment (start 11 0.5) (end 10 0.5) (width 0.508) (layer "B.Cu") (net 1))
 (segment (start -18.5 16) (end -18.5 26) (width 0.508) (layer "B.Cu") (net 17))
 (segment (start 6.5 23.5) (end -4.106 23.5) (width 0.508) (layer "B.Cu") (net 17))
 (segment (start -17.512835 26.987165) (end -16.182 26.987165) (width 0.508) (layer "B.Cu") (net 17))
 (segment (start -17 14.5) (end -18.5 16) (width 0.508) (layer "B.Cu") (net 17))
 (segment (start -4.106 23.5) (end -13.106 14.5) (width 0.508) (layer "B.Cu") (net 17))
 (segment (start -18.5 26) (end -17.512835 26.987165) (width 0.508) (layer "B.Cu") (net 17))
 (segment (start -13.106 14.5) (end -17 14.5) (width 0.508) (layer "B.Cu") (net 17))
 (segment (start 6 -0.25) (end 6 -2.975) (width 0.508) (layer "F.Cu") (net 24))
 (segment (start 2 -0.25) (end 2 -2.975) (width 0.508) (layer "F.Cu") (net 2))
 (segment (start -2 -2.975) (end -2 -0.25) (width 0.508) (layer "F.Cu") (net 4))
 (segment (start -6 -0.25) (end -6 -2.975) (width 0.508) (layer "F.Cu") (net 26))
 (segment (start 18.208 2.292) (end 14 6.5) (width 0.508) (layer "F.Cu") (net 5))
 (segment (start 2.708 -8.708) (end 16.793264 -8.708) (width 0.508) (layer "F.Cu") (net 5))
 (segment (start -2 1.75) (end -0.75 1.75) (width 0.508) (layer "F.Cu") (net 5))
 (segment (start 0 1) (end 0 -6) (width 0.508) (layer "F.Cu") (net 5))
 (segment (start 18.208 -7.293264) (end 18.208 2.292) (width 0.508) (layer "F.Cu") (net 5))
 (segment (start 16.793264 -8.708) (end 18.208 -7.293264) (width 0.508) (layer "F.Cu") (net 5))
 (segment (start 0 -6) (end 2.708 -8.708) (width 0.508) (layer "F.Cu") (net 5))
 (segment (start 14 6.5) (end 11 6.5) (width 0.508) (layer "F.Cu") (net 5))
 (segment (start -0.75 1.75) (end 0 1) (width 0.508) (layer "F.Cu") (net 5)))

